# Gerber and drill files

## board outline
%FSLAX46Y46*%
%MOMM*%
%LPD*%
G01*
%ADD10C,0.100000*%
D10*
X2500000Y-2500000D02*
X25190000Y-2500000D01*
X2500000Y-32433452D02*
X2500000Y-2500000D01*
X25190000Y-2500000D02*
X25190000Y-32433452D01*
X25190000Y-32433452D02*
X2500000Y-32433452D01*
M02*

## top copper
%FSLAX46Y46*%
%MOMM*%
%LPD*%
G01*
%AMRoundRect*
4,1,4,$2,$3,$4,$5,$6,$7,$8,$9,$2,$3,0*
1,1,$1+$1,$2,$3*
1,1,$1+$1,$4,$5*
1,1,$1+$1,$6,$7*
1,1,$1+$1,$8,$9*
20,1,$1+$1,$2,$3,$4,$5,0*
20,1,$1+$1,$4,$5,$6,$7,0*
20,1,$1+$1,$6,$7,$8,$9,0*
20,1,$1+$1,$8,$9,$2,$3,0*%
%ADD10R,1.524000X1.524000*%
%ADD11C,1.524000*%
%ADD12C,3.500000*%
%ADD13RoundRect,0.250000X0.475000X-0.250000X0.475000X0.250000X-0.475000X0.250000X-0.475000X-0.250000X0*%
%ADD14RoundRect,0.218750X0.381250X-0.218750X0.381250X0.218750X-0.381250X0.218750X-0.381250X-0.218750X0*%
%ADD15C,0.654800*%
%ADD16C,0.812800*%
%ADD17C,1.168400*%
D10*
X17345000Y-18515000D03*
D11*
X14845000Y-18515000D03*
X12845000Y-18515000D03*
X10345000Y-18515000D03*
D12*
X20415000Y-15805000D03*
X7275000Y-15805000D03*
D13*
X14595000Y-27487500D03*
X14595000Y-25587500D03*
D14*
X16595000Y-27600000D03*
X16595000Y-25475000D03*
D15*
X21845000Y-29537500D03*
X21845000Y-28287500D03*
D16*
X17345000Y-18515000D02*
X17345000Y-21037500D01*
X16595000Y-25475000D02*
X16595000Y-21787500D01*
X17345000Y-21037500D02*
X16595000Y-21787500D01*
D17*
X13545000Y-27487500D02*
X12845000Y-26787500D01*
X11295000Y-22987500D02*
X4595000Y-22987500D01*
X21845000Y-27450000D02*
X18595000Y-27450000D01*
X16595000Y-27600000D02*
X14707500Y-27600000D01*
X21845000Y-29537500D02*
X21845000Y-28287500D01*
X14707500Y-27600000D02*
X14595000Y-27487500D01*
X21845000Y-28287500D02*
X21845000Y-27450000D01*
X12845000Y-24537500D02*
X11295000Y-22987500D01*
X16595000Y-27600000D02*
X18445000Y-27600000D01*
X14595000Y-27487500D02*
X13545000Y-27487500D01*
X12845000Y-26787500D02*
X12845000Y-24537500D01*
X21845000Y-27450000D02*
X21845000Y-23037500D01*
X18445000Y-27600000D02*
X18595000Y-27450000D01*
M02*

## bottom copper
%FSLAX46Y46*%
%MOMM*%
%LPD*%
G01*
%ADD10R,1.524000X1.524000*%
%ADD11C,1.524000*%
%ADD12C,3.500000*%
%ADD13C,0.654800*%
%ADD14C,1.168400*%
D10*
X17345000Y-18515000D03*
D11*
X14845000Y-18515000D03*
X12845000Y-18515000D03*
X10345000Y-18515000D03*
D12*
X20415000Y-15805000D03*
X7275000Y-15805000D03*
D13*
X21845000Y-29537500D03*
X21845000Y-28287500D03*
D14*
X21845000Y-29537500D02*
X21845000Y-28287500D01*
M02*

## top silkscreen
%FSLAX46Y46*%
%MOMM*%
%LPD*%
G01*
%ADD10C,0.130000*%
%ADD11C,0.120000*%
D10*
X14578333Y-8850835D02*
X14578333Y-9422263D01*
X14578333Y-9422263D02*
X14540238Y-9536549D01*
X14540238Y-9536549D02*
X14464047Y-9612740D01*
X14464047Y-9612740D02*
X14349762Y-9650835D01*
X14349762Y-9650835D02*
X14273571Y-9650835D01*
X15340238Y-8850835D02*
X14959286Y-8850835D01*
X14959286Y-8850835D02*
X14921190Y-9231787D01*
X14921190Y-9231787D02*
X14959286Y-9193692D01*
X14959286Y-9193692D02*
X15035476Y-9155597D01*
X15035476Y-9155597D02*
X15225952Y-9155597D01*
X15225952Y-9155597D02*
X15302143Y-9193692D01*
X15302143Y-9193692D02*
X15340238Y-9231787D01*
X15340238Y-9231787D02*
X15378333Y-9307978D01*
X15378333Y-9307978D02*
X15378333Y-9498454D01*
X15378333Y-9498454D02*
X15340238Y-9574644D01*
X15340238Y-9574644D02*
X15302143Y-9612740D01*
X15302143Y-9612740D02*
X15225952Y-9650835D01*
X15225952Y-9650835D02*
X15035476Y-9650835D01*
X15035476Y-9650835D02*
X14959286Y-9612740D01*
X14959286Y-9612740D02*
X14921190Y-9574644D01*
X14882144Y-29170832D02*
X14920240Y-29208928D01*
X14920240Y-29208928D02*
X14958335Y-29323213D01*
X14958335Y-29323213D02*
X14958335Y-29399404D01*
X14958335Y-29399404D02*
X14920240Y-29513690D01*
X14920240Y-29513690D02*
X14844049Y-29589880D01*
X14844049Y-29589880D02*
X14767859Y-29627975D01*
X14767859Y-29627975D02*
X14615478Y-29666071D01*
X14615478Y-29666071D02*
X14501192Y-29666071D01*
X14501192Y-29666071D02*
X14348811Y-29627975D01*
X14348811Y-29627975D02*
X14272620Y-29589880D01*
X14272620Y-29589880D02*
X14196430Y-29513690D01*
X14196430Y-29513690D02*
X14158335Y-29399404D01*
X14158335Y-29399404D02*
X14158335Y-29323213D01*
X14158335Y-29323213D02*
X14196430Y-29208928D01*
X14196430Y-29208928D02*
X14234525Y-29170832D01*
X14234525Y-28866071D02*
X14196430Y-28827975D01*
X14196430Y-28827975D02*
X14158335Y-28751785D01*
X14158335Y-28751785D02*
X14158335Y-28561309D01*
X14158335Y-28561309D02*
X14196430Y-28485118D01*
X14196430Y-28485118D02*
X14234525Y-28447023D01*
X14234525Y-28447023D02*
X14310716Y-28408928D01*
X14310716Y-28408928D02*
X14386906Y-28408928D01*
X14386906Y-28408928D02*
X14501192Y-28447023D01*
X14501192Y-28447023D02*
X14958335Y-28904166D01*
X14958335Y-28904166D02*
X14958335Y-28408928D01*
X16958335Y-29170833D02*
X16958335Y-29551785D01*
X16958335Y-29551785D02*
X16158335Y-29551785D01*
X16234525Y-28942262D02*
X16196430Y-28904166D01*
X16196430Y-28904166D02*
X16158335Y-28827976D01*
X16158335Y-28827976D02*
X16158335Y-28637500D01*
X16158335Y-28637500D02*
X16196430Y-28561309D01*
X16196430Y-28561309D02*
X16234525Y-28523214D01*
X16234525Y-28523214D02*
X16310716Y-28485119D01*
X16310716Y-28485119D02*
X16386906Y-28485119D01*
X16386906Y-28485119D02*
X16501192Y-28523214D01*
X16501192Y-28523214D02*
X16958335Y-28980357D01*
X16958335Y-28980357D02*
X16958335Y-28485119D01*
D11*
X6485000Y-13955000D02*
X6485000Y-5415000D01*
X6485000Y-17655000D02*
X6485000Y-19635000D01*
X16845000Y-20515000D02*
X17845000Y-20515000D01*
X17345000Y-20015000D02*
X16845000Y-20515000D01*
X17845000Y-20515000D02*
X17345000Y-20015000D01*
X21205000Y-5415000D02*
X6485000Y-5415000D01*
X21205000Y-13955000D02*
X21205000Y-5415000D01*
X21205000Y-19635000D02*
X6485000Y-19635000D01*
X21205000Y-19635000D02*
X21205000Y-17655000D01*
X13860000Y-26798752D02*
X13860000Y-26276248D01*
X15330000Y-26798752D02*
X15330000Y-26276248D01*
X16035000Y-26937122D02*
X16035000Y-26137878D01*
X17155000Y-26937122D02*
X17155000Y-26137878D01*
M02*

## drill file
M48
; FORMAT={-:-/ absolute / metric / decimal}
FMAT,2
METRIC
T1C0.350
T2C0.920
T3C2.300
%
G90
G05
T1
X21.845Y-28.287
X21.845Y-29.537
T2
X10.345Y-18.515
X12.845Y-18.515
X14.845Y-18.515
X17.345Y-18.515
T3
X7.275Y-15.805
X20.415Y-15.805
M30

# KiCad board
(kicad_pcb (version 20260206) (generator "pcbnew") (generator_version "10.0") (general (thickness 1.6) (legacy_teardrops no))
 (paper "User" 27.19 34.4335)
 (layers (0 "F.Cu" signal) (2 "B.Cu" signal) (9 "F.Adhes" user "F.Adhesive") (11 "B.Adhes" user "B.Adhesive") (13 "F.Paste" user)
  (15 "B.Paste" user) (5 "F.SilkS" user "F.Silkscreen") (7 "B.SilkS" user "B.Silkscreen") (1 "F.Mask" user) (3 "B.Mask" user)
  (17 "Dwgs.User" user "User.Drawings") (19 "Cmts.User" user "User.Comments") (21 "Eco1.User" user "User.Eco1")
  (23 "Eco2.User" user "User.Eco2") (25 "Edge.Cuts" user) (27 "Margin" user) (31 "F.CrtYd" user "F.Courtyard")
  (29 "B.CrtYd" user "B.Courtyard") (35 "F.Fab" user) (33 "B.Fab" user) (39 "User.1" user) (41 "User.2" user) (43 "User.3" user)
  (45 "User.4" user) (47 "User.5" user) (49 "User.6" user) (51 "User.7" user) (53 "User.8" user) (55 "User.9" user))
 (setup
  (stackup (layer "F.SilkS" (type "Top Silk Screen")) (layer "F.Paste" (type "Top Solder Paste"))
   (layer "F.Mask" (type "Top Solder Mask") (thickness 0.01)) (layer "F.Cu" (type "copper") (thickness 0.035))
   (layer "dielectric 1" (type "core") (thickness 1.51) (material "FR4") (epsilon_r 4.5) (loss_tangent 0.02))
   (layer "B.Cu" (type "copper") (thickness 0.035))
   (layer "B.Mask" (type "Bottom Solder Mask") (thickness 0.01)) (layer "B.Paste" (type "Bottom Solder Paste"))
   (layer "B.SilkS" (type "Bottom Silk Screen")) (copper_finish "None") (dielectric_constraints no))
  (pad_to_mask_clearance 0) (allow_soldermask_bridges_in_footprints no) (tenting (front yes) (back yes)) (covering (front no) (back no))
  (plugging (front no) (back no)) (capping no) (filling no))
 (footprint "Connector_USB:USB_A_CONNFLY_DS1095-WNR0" (layer "F.Cu") (at 17.345 18.515 180)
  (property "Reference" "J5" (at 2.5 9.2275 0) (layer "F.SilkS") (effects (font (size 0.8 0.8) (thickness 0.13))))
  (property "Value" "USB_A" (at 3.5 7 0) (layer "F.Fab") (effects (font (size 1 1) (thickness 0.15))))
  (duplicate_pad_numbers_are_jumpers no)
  (fp_line (start 10.86 4.56) (end 10.86 13.1) (stroke (width 0.12) (type solid)) (layer "F.SilkS"))
  (fp_line (start 10.86 0.86) (end 10.86 -1.12) (stroke (width 0.12) (type solid)) (layer "F.SilkS"))
  (fp_line (start 0.5 -2) (end -0.5 -2) (stroke (width 0.12) (type solid)) (layer "F.SilkS"))
  (fp_line (start 0 -1.5) (end 0.5 -2) (stroke (width 0.12) (type solid)) (layer "F.SilkS"))
  (fp_line (start -0.5 -2) (end 0 -1.5) (stroke (width 0.12) (type solid)) (layer "F.SilkS"))
  (fp_line (start -3.86 13.1) (end 10.86 13.1) (stroke (width 0.12) (type solid)) (layer "F.SilkS"))
  (fp_line (start -3.86 4.56) (end -3.86 13.1) (stroke (width 0.12) (type solid)) (layer "F.SilkS"))
  (fp_line (start -3.86 -1.12) (end 10.86 -1.12) (stroke (width 0.12) (type solid)) (layer "F.SilkS"))
  (fp_line (start -3.86 -1.12) (end -3.86 0.86) (stroke (width 0.12) (type solid)) (layer "F.SilkS"))
  (pad "1" thru_hole rect (at 0 0 180) (size 1.524 1.524) (drill 0.92) (layers "*.Cu" "*.Mask") (remove_unused_layers no)
   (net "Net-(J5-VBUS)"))
  (pad "2" thru_hole circle (at 2.5 0 180) (size 1.524 1.524) (drill 0.92) (layers "*.Cu" "*.Mask") (remove_unused_layers no) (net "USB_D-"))
  (pad "3" thru_hole circle (at 4.5 0 180) (size 1.524 1.524) (drill 0.92) (layers "*.Cu" "*.Mask") (remove_unused_layers no) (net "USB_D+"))
  (pad "4" thru_hole circle (at 7 0 180) (size 1.524 1.524) (drill 0.92) (layers "*.Cu" "*.Mask") (remove_unused_layers no) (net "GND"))
  (pad "5" thru_hole circle (at -3.07 2.71 180) (size 3.5 3.5) (drill 2.3) (layers "*.Cu" "*.Mask") (remove_unused_layers no) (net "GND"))
  (pad "5" thru_hole circle (at 10.07 2.71 180) (size 3.5 3.5) (drill 2.3) (layers "*.Cu" "*.Mask") (remove_unused_layers no) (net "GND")))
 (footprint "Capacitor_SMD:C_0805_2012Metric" (layer "F.Cu") (at 14.595 26.5375 90)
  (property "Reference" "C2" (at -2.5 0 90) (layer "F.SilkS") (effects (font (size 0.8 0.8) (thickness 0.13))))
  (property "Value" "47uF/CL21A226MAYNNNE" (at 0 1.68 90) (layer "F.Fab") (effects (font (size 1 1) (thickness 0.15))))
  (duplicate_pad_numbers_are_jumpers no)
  (fp_line (start -0.261252 -0.735) (end 0.261252 -0.735) (stroke (width 0.12) (type solid)) (layer "F.SilkS"))
  (fp_line (start -0.261252 0.735) (end 0.261252 0.735) (stroke (width 0.12) (type solid)) (layer "F.SilkS"))
  (pad "1" smd roundrect (at -0.95 0 90) (size 1 1.45) (layers "F.Cu" "F.Mask" "F.Paste") (roundrect_rratio 0.25) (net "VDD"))
  (pad "2" smd roundrect (at 0.95 0 90) (size 1 1.45) (layers "F.Cu" "F.Mask" "F.Paste") (roundrect_rratio 0.25) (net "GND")))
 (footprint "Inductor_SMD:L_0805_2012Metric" (layer "F.Cu") (at 16.595 26.5375 90)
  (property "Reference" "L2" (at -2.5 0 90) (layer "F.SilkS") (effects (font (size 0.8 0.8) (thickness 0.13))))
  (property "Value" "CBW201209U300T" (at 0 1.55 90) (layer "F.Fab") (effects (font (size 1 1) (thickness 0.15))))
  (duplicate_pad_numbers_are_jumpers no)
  (fp_line (start -0.399622 -0.56) (end 0.399622 -0.56) (stroke (width 0.12) (type solid)) (layer "F.SilkS"))
  (fp_line (start -0.399622 0.56) (end 0.399622 0.56) (stroke (width 0.12) (type solid)) (layer "F.SilkS"))
  (pad "1" smd roundrect (at -1.0625 0 90) (size 0.875 1.2) (layers "F.Cu" "F.Mask" "F.Paste") (roundrect_rratio 0.25) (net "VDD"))
  (pad "2" smd roundrect (at 1.0625 0 90) (size 0.875 1.2) (layers "F.Cu" "F.Mask" "F.Paste") (roundrect_rratio 0.25) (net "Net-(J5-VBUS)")))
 (gr_line (start 2.5 2.5) (end 25.19 2.5) (stroke (width 0.1) (type default)) (layer "Edge.Cuts"))
 (gr_line (start 2.5 32.433452) (end 2.5 2.5) (stroke (width 0.1) (type default)) (layer "Edge.Cuts"))
 (gr_line (start 25.19 2.5) (end 25.19 32.433452) (stroke (width 0.1) (type default)) (layer "Edge.Cuts"))
 (gr_line (start 25.19 32.433452) (end 2.5 32.433452) (stroke (width 0.1) (type default)) (layer "Edge.Cuts"))
 (segment (start 17.345 18.515) (end 17.345 21.0375) (width 0.8128) (layer "F.Cu") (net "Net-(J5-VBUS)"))
 (segment (start 16.595 25.475) (end 16.595 21.7875) (width 0.8128) (layer "F.Cu") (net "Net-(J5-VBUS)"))
 (segment (start 17.345 21.0375) (end 16.595 21.7875) (width 0.8128) (layer "F.Cu") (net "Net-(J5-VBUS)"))
 (segment (start 13.545 27.4875) (end 12.845 26.7875) (width 1.1684) (layer "F.Cu") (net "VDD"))
 (segment (start 11.295 22.9875) (end 4.595 22.9875) (width 1.1684) (layer "F.Cu") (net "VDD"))
 (segment (start 21.845 27.45) (end 18.595 27.45) (width 1.1684) (layer "F.Cu") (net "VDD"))
 (segment (start 16.595 27.6) (end 14.7075 27.6) (width 1.1684) (layer "F.Cu") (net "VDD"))
 (segment (start 21.845 29.5375) (end 21.845 28.2875) (width 1.1684) (layer "F.Cu") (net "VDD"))
 (segment (start 14.7075 27.6) (end 14.595 27.4875) (width 1.1684) (layer "F.Cu") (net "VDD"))
 (segment (start 21.845 28.2875) (end 21.845 27.45) (width 1.1684) (layer "F.Cu") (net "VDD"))
 (segment (start 12.845 24.5375) (end 11.295 22.9875) (width 1.1684) (layer "F.Cu") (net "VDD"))
 (segment (start 16.595 27.6) (end 18.445 27.6) (width 1.1684) (layer "F.Cu") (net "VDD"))
 (segment (start 14.595 27.4875) (end 13.545 27.4875) (width 1.1684) (layer "F.Cu") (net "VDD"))
 (segment (start 12.845 26.7875) (end 12.845 24.5375) (width 1.1684) (layer "F.Cu") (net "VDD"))
 (segment (start 21.845 27.45) (end 21.845 23.0375) (width 1.1684) (layer "F.Cu") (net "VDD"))
 (segment (start 18.445 27.6) (end 18.595 27.45) (width 1.1684) (layer "F.Cu") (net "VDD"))
 (via (at 21.845 29.5375) (size 0.6548) (drill 0.35) (layers "F.Cu" "B.Cu") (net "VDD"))
 (via (at 21.845 28.2875) (size 0.6548) (drill 0.35) (layers "F.Cu" "B.Cu") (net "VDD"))
 (segment (start 21.845 29.5375) (end 21.845 28.2875) (width 1.1684) (layer "B.Cu") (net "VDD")))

